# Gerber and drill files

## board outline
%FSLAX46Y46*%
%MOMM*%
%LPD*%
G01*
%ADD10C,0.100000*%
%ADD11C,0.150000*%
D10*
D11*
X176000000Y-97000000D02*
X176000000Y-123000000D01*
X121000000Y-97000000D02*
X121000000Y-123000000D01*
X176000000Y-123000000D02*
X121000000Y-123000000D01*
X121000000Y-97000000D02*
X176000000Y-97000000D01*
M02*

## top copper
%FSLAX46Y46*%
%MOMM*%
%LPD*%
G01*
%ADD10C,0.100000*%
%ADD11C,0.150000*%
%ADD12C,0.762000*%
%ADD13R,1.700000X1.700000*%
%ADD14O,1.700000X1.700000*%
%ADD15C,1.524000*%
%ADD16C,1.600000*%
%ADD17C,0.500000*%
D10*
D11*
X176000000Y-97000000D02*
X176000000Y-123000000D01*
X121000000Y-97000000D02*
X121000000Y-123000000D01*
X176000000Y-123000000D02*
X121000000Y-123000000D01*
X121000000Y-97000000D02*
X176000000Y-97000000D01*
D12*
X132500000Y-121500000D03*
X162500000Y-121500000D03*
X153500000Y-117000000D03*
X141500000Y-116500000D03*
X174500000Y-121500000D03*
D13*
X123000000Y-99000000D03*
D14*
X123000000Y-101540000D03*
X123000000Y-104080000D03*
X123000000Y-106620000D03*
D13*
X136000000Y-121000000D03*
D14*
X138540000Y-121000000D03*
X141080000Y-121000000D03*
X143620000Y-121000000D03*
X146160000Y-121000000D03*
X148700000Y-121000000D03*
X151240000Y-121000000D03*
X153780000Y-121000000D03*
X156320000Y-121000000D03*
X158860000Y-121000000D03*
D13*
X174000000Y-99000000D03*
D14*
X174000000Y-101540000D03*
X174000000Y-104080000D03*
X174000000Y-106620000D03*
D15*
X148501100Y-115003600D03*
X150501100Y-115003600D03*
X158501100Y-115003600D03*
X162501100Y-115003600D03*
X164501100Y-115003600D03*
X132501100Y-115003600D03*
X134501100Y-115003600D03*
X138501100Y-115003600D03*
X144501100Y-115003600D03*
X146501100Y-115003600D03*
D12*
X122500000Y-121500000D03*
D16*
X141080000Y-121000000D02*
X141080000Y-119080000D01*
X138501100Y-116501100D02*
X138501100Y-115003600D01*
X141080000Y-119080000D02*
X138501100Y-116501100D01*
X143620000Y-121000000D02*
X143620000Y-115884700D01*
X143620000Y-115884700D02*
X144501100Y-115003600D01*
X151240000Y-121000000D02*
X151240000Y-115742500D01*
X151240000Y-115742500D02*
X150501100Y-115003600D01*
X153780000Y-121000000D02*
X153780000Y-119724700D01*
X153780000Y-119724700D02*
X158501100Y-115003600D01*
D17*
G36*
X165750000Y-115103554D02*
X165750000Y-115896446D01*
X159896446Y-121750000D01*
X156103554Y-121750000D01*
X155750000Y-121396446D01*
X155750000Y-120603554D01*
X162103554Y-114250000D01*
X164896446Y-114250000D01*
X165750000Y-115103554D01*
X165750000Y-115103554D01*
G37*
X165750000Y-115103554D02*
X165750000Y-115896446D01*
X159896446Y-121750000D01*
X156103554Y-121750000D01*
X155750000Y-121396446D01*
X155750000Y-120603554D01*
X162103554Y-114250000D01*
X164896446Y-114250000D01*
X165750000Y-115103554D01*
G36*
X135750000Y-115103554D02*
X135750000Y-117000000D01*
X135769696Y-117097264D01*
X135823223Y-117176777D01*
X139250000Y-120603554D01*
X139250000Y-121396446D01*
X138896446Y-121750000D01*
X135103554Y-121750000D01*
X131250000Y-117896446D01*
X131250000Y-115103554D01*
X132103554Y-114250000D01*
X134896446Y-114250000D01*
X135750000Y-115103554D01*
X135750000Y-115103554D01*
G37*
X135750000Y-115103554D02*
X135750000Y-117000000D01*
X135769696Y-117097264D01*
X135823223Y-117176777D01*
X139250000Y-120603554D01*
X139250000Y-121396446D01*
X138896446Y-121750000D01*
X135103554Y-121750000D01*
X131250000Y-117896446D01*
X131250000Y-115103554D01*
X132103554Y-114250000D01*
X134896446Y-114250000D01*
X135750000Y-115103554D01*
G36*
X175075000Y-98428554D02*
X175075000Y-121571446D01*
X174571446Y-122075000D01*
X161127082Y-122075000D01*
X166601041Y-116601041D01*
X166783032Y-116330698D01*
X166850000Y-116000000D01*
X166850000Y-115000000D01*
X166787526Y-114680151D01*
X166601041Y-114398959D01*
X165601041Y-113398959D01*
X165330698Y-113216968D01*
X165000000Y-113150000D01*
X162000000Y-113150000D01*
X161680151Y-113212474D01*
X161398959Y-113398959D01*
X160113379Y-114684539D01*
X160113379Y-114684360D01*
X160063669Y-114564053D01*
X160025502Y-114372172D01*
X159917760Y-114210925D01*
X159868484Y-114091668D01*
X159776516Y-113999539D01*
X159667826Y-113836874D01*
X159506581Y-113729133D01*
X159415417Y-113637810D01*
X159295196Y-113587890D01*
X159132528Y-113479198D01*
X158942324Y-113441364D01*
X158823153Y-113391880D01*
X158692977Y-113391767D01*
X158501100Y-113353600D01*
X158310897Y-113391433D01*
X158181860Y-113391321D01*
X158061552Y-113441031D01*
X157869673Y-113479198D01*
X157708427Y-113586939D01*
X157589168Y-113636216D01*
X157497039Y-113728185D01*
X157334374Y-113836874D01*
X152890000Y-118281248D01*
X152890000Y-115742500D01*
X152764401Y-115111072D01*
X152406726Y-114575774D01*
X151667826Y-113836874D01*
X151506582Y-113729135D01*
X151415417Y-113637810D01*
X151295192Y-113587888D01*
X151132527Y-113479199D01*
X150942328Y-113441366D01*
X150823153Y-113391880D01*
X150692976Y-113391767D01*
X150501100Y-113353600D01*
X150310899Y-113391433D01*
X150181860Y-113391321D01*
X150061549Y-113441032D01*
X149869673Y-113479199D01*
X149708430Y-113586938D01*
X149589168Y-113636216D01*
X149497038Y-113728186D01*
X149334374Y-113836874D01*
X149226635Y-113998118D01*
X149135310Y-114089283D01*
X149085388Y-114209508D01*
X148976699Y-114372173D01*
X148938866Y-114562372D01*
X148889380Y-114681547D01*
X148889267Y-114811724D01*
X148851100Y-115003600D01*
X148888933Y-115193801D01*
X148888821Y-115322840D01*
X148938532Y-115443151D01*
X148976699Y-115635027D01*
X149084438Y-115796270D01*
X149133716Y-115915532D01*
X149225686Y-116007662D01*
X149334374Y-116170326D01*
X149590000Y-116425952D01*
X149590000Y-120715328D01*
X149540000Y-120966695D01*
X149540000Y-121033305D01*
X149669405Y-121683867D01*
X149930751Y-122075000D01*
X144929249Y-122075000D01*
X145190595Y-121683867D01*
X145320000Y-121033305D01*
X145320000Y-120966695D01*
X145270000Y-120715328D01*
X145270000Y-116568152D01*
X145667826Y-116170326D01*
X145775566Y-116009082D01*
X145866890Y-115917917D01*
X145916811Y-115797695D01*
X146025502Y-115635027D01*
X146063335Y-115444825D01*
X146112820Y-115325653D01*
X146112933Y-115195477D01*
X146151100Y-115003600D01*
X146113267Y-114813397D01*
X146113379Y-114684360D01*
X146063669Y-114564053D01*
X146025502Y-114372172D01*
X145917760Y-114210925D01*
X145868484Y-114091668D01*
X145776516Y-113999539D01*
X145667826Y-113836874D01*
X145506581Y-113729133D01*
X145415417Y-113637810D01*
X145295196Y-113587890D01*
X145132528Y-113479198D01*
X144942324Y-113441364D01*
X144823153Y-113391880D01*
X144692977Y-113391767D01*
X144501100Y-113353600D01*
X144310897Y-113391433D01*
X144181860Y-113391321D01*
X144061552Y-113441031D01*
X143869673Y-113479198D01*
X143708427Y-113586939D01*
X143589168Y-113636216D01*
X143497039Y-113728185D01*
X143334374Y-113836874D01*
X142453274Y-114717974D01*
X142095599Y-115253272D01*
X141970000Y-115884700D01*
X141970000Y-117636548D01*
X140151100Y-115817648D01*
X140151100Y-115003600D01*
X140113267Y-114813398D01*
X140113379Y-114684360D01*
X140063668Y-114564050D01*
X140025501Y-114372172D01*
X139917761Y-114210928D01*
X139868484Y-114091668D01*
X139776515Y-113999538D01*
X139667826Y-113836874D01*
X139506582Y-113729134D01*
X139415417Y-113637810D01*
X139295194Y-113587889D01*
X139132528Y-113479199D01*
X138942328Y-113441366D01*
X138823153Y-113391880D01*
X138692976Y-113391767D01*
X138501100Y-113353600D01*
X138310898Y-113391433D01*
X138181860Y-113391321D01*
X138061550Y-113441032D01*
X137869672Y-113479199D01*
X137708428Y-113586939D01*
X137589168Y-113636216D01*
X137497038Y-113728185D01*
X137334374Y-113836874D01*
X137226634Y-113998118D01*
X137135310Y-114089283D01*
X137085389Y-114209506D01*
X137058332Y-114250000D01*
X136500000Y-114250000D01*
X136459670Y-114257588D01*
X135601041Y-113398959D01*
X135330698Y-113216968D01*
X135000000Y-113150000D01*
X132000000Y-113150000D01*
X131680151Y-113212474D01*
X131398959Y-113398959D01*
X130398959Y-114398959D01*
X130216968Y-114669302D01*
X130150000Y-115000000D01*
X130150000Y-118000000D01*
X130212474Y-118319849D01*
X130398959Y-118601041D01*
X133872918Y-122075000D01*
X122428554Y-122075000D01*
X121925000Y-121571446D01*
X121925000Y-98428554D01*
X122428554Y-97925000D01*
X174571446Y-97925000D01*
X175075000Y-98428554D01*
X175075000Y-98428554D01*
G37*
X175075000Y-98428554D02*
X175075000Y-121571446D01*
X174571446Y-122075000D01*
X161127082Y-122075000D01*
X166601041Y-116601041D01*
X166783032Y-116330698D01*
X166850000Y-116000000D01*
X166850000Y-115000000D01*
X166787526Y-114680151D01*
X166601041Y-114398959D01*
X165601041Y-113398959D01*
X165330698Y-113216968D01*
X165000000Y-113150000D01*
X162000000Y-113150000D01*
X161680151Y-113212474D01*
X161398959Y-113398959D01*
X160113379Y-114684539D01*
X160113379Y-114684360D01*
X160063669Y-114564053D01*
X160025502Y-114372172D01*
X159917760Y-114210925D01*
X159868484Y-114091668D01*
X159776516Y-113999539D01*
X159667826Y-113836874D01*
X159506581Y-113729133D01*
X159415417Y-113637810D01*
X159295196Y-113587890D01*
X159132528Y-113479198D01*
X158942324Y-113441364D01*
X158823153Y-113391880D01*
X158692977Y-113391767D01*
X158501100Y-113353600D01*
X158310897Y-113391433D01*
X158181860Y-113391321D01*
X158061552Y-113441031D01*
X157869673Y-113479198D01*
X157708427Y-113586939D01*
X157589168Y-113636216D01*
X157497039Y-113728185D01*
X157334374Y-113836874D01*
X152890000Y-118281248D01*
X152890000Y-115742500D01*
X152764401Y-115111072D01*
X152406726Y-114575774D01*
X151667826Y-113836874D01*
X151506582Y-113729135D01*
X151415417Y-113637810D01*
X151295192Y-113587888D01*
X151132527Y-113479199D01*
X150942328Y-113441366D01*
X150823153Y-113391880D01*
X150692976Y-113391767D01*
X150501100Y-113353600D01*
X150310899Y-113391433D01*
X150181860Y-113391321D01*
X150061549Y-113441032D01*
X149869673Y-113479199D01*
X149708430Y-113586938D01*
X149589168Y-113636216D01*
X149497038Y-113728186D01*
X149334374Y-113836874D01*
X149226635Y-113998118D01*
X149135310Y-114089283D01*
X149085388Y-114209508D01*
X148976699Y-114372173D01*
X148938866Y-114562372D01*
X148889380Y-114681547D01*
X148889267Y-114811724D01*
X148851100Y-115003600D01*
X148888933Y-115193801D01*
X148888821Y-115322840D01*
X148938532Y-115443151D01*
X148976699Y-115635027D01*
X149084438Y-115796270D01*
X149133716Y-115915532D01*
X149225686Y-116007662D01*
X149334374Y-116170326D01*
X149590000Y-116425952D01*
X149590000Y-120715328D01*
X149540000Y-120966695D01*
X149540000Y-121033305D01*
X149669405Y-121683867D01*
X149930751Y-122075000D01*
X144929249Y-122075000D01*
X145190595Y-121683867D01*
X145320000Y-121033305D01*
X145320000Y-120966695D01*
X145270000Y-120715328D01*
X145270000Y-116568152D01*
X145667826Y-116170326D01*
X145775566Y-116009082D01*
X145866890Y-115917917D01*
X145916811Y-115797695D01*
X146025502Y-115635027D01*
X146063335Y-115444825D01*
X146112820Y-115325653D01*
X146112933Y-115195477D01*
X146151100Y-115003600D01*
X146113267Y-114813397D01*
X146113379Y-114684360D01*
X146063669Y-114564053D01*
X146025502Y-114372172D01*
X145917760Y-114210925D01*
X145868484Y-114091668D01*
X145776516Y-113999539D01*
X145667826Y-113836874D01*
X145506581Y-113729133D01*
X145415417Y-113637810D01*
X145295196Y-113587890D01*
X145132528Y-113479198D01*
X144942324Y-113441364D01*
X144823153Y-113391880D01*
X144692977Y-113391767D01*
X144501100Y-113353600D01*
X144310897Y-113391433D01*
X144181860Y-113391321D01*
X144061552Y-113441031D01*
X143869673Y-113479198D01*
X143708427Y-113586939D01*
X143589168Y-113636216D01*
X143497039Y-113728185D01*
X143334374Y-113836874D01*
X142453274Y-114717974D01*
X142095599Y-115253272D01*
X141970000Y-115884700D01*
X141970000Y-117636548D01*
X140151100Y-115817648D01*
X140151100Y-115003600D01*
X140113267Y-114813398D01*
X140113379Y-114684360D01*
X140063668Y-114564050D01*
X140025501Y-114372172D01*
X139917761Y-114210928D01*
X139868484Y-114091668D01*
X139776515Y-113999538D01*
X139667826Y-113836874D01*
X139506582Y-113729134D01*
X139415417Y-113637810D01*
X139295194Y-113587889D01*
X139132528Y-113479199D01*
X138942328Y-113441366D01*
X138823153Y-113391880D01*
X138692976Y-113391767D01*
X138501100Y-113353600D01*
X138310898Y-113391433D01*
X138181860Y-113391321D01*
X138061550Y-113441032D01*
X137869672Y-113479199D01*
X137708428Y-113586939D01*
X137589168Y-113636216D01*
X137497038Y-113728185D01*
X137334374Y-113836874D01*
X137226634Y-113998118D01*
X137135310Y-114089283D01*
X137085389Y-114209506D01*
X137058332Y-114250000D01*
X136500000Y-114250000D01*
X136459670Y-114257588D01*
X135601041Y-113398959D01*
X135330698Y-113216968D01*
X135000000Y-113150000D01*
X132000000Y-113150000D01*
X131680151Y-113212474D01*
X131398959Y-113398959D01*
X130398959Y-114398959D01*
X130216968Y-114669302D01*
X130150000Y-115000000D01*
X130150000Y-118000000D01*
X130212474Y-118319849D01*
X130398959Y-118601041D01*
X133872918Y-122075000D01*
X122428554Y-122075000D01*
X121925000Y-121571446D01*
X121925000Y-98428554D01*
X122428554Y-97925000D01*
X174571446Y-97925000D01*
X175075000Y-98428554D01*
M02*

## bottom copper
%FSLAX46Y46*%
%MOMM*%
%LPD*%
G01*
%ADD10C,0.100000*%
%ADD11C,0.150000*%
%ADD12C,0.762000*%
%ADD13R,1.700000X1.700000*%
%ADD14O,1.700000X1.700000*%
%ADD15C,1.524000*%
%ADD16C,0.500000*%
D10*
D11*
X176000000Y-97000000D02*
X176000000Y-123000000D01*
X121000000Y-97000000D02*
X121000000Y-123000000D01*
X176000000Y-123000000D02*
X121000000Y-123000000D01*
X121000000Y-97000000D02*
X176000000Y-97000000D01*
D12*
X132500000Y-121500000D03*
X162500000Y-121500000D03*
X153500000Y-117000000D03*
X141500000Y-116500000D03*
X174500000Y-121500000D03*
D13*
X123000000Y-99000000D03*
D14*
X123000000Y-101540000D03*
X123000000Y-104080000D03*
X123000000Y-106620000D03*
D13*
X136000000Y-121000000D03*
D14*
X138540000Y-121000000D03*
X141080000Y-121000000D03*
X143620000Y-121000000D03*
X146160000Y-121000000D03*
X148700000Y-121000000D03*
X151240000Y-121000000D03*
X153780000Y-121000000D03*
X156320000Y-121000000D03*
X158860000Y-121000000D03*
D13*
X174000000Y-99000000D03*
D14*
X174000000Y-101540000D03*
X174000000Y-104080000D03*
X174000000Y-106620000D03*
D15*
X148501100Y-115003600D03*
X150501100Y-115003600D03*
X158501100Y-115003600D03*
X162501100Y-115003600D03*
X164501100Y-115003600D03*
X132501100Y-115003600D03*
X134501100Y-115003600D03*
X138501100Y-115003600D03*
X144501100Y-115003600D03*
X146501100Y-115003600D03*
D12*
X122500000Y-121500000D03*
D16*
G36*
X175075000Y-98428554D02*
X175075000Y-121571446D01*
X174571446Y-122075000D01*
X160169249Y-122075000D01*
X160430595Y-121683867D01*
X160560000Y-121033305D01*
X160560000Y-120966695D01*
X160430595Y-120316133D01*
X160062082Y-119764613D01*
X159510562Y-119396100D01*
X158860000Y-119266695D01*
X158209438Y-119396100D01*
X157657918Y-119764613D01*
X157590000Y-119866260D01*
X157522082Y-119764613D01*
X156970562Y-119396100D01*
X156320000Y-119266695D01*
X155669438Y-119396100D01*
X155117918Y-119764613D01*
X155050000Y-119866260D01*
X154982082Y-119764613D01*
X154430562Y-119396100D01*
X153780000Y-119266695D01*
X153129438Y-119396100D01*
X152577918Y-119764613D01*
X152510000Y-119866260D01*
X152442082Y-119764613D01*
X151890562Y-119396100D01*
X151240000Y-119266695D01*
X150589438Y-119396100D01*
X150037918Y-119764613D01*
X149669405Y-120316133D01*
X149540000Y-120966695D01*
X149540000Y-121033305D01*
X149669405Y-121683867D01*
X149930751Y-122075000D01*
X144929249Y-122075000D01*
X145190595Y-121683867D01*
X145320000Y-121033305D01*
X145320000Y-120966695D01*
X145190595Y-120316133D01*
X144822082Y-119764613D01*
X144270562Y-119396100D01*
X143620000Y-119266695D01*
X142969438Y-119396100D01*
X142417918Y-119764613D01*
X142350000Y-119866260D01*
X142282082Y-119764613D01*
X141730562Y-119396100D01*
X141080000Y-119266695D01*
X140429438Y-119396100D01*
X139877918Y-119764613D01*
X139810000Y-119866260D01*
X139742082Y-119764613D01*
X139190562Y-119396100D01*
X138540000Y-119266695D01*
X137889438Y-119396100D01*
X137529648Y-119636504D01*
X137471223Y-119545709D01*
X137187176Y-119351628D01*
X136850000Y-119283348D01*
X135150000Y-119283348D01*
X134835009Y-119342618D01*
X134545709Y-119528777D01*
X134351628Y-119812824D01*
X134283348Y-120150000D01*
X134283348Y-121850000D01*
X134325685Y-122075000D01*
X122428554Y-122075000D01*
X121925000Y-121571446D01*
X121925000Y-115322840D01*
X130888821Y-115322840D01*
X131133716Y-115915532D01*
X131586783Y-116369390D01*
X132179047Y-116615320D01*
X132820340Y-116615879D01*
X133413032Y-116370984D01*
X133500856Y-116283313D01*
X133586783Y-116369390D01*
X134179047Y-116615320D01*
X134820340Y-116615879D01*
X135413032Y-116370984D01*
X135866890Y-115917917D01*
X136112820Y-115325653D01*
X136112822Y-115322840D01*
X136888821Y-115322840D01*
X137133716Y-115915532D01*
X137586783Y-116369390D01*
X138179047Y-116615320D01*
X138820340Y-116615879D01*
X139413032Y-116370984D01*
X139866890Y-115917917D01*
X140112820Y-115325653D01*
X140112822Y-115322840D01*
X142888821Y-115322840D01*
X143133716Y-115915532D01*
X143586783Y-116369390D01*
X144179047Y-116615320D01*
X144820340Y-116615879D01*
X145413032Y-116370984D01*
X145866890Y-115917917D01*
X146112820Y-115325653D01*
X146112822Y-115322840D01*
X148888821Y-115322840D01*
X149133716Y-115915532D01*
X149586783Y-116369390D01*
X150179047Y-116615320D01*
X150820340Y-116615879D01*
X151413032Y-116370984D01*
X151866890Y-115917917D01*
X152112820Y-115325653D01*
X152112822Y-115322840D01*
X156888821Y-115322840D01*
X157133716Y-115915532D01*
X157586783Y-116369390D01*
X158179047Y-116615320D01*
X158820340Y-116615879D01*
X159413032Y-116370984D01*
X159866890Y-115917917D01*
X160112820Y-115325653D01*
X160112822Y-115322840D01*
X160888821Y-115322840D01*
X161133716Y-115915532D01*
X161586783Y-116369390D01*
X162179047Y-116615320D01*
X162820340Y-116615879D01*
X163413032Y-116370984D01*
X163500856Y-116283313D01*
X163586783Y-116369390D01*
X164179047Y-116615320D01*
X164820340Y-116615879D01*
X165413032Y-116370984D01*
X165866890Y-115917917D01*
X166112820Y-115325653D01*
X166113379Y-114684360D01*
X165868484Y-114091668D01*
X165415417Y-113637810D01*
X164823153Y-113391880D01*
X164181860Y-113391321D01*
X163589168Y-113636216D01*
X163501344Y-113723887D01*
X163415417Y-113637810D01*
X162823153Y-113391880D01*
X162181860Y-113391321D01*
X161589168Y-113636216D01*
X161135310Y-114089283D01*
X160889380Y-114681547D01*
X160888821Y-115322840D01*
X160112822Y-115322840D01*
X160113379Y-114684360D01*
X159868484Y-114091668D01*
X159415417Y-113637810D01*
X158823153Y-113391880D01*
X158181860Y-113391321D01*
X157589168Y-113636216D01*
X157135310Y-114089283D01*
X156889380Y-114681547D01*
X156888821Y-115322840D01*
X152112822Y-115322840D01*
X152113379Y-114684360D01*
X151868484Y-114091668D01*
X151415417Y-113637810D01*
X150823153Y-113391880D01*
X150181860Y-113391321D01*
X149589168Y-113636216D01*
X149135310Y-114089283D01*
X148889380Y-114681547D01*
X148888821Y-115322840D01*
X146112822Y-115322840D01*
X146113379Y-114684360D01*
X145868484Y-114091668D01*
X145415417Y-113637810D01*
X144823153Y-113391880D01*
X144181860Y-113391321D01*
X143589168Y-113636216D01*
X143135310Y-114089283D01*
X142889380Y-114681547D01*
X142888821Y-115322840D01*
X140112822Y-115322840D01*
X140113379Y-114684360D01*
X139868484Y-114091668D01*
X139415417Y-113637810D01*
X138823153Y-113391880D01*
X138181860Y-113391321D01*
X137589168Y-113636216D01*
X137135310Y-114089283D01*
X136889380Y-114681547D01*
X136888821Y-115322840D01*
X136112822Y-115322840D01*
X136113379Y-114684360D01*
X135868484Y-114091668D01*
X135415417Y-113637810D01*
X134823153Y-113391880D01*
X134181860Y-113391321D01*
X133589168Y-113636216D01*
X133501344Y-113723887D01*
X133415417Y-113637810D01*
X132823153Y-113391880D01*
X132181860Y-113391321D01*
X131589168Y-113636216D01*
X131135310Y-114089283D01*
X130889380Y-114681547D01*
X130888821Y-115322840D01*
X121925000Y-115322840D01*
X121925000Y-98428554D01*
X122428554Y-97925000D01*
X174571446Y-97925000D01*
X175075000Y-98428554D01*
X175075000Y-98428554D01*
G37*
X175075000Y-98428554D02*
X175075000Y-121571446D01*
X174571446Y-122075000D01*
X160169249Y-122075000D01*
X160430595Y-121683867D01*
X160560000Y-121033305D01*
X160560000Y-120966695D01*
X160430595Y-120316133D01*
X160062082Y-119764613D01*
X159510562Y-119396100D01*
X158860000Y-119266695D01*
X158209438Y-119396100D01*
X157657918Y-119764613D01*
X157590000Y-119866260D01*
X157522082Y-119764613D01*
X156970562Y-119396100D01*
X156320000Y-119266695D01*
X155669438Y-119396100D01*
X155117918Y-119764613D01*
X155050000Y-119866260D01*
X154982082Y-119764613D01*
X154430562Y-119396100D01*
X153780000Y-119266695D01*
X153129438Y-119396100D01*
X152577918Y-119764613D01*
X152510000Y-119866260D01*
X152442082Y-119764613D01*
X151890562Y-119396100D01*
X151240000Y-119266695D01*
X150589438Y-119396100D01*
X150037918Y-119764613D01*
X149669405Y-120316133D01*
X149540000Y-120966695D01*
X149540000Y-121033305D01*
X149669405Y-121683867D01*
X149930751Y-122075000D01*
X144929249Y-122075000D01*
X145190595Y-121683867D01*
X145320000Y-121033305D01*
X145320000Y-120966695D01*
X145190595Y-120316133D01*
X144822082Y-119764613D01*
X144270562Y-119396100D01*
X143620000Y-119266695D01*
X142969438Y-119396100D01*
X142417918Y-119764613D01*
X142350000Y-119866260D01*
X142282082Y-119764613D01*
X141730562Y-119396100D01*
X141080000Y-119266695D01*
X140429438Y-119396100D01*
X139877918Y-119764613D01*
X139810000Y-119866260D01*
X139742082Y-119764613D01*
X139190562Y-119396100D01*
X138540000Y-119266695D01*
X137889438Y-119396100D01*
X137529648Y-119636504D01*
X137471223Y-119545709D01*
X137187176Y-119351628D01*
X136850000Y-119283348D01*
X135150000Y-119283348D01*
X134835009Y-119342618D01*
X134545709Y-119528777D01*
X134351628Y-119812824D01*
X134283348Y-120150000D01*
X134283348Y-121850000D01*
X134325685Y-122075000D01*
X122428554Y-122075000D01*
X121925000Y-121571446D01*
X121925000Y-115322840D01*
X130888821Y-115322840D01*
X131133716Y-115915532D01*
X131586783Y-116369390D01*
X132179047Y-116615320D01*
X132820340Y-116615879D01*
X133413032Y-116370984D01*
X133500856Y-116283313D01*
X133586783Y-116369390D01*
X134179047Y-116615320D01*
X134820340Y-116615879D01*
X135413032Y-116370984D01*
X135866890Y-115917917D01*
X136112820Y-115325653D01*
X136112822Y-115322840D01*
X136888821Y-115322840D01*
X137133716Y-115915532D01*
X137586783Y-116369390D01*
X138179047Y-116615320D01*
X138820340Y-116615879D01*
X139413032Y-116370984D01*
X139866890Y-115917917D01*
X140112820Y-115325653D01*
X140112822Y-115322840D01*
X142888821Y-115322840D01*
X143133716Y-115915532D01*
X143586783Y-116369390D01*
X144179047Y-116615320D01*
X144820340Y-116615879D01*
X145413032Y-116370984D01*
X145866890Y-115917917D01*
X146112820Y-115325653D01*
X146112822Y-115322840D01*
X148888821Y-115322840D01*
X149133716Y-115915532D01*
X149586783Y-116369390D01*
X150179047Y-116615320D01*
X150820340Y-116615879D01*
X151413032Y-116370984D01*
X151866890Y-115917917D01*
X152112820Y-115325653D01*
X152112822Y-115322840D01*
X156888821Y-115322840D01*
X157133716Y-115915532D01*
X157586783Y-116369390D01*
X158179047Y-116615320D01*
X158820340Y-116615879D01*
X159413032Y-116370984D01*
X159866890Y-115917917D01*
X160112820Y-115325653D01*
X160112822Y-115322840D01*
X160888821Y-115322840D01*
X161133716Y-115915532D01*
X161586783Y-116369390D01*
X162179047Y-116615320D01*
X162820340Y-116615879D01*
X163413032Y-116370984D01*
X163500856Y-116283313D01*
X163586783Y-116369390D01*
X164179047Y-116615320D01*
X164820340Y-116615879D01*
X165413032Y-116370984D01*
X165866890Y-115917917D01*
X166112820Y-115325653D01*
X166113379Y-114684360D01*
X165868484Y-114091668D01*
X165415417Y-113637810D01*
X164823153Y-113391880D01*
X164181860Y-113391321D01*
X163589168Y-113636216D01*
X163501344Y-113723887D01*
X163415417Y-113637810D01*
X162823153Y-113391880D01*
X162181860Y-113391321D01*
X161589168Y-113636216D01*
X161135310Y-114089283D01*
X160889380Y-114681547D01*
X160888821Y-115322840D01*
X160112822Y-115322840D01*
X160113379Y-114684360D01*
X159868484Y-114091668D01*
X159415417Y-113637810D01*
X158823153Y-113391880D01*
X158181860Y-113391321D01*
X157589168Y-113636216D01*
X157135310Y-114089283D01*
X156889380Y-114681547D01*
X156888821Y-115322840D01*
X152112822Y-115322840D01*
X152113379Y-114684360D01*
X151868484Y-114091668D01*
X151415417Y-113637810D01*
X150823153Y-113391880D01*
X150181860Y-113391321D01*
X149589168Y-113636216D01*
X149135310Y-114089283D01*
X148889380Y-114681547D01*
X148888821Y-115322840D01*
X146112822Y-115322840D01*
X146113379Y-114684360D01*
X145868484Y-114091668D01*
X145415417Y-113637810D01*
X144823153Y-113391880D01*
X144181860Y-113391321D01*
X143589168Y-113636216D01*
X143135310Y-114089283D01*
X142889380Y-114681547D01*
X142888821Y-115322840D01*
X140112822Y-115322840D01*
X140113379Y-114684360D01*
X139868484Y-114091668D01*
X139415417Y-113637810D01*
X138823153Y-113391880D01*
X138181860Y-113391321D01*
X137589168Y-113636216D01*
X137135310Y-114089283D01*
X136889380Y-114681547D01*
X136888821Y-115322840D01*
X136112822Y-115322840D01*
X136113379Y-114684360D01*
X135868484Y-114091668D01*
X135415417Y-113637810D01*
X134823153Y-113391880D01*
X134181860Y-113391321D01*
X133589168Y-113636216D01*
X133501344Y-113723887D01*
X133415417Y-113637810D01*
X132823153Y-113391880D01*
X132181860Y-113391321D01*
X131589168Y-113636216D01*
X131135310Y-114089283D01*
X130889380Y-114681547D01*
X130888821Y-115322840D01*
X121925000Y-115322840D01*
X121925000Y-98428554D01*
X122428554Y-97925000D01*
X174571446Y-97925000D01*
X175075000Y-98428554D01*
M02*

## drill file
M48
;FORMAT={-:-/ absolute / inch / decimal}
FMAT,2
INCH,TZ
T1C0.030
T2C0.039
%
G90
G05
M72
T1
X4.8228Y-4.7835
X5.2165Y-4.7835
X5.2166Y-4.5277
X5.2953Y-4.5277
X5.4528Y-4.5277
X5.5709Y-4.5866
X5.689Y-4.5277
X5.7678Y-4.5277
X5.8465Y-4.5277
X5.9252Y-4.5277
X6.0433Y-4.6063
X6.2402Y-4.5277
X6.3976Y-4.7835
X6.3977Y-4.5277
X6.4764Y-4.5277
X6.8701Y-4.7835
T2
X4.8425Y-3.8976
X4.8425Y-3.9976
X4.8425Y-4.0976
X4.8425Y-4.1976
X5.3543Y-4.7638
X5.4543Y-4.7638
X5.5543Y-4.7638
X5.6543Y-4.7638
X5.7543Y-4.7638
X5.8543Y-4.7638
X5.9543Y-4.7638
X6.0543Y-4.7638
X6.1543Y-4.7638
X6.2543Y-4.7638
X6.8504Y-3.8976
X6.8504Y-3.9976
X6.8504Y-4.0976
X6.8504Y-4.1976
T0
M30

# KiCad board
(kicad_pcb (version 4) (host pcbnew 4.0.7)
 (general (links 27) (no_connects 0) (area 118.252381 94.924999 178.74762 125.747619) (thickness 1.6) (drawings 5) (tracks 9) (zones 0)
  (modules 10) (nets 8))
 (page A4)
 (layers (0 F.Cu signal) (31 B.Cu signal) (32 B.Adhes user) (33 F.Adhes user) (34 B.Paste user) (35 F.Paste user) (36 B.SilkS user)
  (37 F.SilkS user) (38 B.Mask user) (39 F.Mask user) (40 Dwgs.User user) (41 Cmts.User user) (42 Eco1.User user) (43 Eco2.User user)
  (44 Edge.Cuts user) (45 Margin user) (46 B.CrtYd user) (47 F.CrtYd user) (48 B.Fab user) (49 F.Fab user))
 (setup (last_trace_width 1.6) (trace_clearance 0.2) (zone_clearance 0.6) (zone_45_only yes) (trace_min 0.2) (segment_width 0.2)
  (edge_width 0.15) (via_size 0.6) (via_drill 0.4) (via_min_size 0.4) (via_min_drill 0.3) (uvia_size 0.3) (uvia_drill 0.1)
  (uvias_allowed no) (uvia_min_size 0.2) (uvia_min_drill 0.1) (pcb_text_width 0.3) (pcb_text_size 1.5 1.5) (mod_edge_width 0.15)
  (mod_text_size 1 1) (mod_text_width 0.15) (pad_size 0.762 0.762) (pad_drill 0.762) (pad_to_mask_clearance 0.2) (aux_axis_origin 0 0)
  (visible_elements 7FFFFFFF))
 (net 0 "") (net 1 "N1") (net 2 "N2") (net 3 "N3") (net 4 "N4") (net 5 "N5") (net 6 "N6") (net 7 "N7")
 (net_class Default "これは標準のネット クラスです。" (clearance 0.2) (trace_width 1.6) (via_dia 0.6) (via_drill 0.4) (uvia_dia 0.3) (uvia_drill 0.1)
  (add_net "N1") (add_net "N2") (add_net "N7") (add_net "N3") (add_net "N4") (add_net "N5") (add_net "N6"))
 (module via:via (layer F.Cu) (at 132.5 121.5)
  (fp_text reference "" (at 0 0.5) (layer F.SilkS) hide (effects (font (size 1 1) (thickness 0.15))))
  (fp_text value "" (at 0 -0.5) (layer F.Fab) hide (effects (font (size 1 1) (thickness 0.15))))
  (pad 1 thru_hole circle (at 0 0) (size 0.762 0.762) (drill 0.762) (layers *.Cu *.Mask) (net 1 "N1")))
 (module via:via (layer F.Cu) (at 162.5 121.5)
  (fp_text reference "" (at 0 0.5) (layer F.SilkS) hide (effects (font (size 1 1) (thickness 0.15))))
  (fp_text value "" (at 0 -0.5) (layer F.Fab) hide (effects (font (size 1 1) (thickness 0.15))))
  (pad 1 thru_hole circle (at 0 0) (size 0.762 0.762) (drill 0.762) (layers *.Cu *.Mask) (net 1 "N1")))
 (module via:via (layer F.Cu) (at 153.5 117)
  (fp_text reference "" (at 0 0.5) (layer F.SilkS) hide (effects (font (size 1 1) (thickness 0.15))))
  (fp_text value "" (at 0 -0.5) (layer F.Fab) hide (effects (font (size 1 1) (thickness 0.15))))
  (pad 1 thru_hole circle (at 0 0) (size 0.762 0.762) (drill 0.762) (layers *.Cu *.Mask) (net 1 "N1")))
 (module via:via (layer F.Cu) (at 141.5 116.5)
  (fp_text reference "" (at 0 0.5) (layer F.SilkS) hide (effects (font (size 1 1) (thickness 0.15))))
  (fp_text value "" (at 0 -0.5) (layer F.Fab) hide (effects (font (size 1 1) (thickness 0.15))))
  (pad 1 thru_hole circle (at 0 0) (size 0.762 0.762) (drill 0.762) (layers *.Cu *.Mask) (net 1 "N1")))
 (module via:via (layer F.Cu) (at 174.5 121.5)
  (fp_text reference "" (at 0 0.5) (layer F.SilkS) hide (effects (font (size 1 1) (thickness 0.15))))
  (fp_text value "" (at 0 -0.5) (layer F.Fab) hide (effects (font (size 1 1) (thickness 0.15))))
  (pad 1 thru_hole circle (at 0 0) (size 0.762 0.762) (drill 0.762) (layers *.Cu *.Mask) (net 1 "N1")))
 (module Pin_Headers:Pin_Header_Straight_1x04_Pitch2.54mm (layer F.Cu) (at 123 99)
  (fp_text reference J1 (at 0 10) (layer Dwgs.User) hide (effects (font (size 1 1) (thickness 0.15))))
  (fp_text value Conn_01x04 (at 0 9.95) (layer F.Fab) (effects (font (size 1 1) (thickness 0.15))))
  (pad 1 thru_hole rect (at 0 0) (size 1.7 1.7) (drill 1) (layers *.Cu *.Mask) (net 1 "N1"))
  (pad 2 thru_hole oval (at 0 2.54) (size 1.7 1.7) (drill 1) (layers *.Cu *.Mask) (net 1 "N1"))
  (pad 3 thru_hole oval (at 0 5.08) (size 1.7 1.7) (drill 1) (layers *.Cu *.Mask) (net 1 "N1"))
  (pad 4 thru_hole oval (at 0 7.62) (size 1.7 1.7) (drill 1) (layers *.Cu *.Mask) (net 1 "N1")))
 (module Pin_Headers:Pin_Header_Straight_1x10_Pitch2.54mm (layer F.Cu) (at 136 121 90)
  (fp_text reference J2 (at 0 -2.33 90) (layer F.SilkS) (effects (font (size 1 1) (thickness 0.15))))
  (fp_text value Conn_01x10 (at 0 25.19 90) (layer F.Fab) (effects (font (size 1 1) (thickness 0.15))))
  (pad 1 thru_hole rect (at 0 0 90) (size 1.7 1.7) (drill 1) (layers *.Cu *.Mask) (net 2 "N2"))
  (pad 2 thru_hole oval (at 0 2.54 90) (size 1.7 1.7) (drill 1) (layers *.Cu *.Mask) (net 2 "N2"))
  (pad 3 thru_hole oval (at 0 5.08 90) (size 1.7 1.7) (drill 1) (layers *.Cu *.Mask) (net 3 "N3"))
  (pad 4 thru_hole oval (at 0 7.62 90) (size 1.7 1.7) (drill 1) (layers *.Cu *.Mask) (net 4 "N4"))
  (pad 5 thru_hole oval (at 0 10.16 90) (size 1.7 1.7) (drill 1) (layers *.Cu *.Mask) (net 1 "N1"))
  (pad 6 thru_hole oval (at 0 12.7 90) (size 1.7 1.7) (drill 1) (layers *.Cu *.Mask) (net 1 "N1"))
  (pad 7 thru_hole oval (at 0 15.24 90) (size 1.7 1.7) (drill 1) (layers *.Cu *.Mask) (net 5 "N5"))
  (pad 8 thru_hole oval (at 0 17.78 90) (size 1.7 1.7) (drill 1) (layers *.Cu *.Mask) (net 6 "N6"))
  (pad 9 thru_hole oval (at 0 20.32 90) (size 1.7 1.7) (drill 1) (layers *.Cu *.Mask) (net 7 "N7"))
  (pad 10 thru_hole oval (at 0 22.86 90) (size 1.7 1.7) (drill 1) (layers *.Cu *.Mask) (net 7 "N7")))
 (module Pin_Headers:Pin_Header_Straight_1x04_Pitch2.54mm (layer F.Cu) (at 174 99)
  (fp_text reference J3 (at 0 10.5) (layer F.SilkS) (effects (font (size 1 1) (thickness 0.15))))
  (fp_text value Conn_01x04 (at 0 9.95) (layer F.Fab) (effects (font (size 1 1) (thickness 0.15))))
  (pad 1 thru_hole rect (at 0 0) (size 1.7 1.7) (drill 1) (layers *.Cu *.Mask) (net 1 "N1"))
  (pad 2 thru_hole oval (at 0 2.54) (size 1.7 1.7) (drill 1) (layers *.Cu *.Mask) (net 1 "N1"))
  (pad 3 thru_hole oval (at 0 5.08) (size 1.7 1.7) (drill 1) (layers *.Cu *.Mask) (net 1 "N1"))
  (pad 4 thru_hole oval (at 0 7.62) (size 1.7 1.7) (drill 1) (layers *.Cu *.Mask) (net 1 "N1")))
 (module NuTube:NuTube (layer F.Cu) (at 148.5011 105.0036)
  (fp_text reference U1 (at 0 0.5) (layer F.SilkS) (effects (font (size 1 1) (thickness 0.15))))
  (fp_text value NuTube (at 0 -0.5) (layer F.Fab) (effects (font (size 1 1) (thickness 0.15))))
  (pad 6 thru_hole circle (at 0 10) (size 1.524 1.524) (drill 0.762) (layers *.Cu *.Mask) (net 1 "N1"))
  (pad 7 thru_hole circle (at 2 10) (size 1.524 1.524) (drill 0.762) (layers *.Cu *.Mask) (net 5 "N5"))
  (pad 8 thru_hole circle (at 10 10) (size 1.524 1.524) (drill 0.762) (layers *.Cu *.Mask) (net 6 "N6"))
  (pad 9 thru_hole circle (at 14 10) (size 1.524 1.524) (drill 0.762) (layers *.Cu *.Mask) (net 7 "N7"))
  (pad 10 thru_hole circle (at 16 10) (size 1.524 1.524) (drill 0.762) (layers *.Cu *.Mask) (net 7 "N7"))
  (pad 1 thru_hole circle (at -16 10) (size 1.524 1.524) (drill 0.762) (layers *.Cu *.Mask) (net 2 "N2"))
  (pad 2 thru_hole circle (at -14 10) (size 1.524 1.524) (drill 0.762) (layers *.Cu *.Mask) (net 2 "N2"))
  (pad 3 thru_hole circle (at -10 10) (size 1.524 1.524) (drill 0.762) (layers *.Cu *.Mask) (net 3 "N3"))
  (pad 4 thru_hole circle (at -4 10) (size 1.524 1.524) (drill 0.762) (layers *.Cu *.Mask) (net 4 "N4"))
  (pad 5 thru_hole circle (at -2 10) (size 1.524 1.524) (drill 0.762) (layers *.Cu *.Mask) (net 1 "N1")))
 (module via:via (layer F.Cu) (at 122.5 121.5)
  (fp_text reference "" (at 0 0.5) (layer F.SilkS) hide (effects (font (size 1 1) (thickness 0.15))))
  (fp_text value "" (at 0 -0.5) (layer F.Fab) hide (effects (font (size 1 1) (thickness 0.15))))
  (pad 1 thru_hole circle (at 0 0) (size 0.762 0.762) (drill 0.762) (layers *.Cu *.Mask) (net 1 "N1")))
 (gr_line (start 176 97) (end 176 123) (angle 90) (layer Edge.Cuts) (width 0.15))
 (gr_line (start 121 97) (end 121 123) (angle 90) (layer Edge.Cuts) (width 0.15))
 (gr_line (start 176 123) (end 121 123) (angle 90) (layer Edge.Cuts) (width 0.15))
 (gr_line (start 121 97) (end 176 97) (angle 90) (layer Edge.Cuts) (width 0.15))
 (segment (start 141.08 121) (end 141.08 119.08) (width 1.6) (layer F.Cu) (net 3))
 (segment (start 138.5011 116.5011) (end 138.5011 115.0036) (width 1.6) (layer F.Cu) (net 3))
 (segment (start 141.08 119.08) (end 138.5011 116.5011) (width 1.6) (layer F.Cu) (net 3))
 (segment (start 143.62 121) (end 143.62 115.8847) (width 1.6) (layer F.Cu) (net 4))
 (segment (start 143.62 115.8847) (end 144.5011 115.0036) (width 1.6) (layer F.Cu) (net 4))
 (segment (start 151.24 121) (end 151.24 115.7425) (width 1.6) (layer F.Cu) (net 5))
 (segment (start 151.24 115.7425) (end 150.5011 115.0036) (width 1.6) (layer F.Cu) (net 5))
 (segment (start 153.78 121) (end 153.78 119.7247) (width 1.6) (layer F.Cu) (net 6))
 (segment (start 153.78 119.7247) (end 158.5011 115.0036) (width 1.6) (layer F.Cu) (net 6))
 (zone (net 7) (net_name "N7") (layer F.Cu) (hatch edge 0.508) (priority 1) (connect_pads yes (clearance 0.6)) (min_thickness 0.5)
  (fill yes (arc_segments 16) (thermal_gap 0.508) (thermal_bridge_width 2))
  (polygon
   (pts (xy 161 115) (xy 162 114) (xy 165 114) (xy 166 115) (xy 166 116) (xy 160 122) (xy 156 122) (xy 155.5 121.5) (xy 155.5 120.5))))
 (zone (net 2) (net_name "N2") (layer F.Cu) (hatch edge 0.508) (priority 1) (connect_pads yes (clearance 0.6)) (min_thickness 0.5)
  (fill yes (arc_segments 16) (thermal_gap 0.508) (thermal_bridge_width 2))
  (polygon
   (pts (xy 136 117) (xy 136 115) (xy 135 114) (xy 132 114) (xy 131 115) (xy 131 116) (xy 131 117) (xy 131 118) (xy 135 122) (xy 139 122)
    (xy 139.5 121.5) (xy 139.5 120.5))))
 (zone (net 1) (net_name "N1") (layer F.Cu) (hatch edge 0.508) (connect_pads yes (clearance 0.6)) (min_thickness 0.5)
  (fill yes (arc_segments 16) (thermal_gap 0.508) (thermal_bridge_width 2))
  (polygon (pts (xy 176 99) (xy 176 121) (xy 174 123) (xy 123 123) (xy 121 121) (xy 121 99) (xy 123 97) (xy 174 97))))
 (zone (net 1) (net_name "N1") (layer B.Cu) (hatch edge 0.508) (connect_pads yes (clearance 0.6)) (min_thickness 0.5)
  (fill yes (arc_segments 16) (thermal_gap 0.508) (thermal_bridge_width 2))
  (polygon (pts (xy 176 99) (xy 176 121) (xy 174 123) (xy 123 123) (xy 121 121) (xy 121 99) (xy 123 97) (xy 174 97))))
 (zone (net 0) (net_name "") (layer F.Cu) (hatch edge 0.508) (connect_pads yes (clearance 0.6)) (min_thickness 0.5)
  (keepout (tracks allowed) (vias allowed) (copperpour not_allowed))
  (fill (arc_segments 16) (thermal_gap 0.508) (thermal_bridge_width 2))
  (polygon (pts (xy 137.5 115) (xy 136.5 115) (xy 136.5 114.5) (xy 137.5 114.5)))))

